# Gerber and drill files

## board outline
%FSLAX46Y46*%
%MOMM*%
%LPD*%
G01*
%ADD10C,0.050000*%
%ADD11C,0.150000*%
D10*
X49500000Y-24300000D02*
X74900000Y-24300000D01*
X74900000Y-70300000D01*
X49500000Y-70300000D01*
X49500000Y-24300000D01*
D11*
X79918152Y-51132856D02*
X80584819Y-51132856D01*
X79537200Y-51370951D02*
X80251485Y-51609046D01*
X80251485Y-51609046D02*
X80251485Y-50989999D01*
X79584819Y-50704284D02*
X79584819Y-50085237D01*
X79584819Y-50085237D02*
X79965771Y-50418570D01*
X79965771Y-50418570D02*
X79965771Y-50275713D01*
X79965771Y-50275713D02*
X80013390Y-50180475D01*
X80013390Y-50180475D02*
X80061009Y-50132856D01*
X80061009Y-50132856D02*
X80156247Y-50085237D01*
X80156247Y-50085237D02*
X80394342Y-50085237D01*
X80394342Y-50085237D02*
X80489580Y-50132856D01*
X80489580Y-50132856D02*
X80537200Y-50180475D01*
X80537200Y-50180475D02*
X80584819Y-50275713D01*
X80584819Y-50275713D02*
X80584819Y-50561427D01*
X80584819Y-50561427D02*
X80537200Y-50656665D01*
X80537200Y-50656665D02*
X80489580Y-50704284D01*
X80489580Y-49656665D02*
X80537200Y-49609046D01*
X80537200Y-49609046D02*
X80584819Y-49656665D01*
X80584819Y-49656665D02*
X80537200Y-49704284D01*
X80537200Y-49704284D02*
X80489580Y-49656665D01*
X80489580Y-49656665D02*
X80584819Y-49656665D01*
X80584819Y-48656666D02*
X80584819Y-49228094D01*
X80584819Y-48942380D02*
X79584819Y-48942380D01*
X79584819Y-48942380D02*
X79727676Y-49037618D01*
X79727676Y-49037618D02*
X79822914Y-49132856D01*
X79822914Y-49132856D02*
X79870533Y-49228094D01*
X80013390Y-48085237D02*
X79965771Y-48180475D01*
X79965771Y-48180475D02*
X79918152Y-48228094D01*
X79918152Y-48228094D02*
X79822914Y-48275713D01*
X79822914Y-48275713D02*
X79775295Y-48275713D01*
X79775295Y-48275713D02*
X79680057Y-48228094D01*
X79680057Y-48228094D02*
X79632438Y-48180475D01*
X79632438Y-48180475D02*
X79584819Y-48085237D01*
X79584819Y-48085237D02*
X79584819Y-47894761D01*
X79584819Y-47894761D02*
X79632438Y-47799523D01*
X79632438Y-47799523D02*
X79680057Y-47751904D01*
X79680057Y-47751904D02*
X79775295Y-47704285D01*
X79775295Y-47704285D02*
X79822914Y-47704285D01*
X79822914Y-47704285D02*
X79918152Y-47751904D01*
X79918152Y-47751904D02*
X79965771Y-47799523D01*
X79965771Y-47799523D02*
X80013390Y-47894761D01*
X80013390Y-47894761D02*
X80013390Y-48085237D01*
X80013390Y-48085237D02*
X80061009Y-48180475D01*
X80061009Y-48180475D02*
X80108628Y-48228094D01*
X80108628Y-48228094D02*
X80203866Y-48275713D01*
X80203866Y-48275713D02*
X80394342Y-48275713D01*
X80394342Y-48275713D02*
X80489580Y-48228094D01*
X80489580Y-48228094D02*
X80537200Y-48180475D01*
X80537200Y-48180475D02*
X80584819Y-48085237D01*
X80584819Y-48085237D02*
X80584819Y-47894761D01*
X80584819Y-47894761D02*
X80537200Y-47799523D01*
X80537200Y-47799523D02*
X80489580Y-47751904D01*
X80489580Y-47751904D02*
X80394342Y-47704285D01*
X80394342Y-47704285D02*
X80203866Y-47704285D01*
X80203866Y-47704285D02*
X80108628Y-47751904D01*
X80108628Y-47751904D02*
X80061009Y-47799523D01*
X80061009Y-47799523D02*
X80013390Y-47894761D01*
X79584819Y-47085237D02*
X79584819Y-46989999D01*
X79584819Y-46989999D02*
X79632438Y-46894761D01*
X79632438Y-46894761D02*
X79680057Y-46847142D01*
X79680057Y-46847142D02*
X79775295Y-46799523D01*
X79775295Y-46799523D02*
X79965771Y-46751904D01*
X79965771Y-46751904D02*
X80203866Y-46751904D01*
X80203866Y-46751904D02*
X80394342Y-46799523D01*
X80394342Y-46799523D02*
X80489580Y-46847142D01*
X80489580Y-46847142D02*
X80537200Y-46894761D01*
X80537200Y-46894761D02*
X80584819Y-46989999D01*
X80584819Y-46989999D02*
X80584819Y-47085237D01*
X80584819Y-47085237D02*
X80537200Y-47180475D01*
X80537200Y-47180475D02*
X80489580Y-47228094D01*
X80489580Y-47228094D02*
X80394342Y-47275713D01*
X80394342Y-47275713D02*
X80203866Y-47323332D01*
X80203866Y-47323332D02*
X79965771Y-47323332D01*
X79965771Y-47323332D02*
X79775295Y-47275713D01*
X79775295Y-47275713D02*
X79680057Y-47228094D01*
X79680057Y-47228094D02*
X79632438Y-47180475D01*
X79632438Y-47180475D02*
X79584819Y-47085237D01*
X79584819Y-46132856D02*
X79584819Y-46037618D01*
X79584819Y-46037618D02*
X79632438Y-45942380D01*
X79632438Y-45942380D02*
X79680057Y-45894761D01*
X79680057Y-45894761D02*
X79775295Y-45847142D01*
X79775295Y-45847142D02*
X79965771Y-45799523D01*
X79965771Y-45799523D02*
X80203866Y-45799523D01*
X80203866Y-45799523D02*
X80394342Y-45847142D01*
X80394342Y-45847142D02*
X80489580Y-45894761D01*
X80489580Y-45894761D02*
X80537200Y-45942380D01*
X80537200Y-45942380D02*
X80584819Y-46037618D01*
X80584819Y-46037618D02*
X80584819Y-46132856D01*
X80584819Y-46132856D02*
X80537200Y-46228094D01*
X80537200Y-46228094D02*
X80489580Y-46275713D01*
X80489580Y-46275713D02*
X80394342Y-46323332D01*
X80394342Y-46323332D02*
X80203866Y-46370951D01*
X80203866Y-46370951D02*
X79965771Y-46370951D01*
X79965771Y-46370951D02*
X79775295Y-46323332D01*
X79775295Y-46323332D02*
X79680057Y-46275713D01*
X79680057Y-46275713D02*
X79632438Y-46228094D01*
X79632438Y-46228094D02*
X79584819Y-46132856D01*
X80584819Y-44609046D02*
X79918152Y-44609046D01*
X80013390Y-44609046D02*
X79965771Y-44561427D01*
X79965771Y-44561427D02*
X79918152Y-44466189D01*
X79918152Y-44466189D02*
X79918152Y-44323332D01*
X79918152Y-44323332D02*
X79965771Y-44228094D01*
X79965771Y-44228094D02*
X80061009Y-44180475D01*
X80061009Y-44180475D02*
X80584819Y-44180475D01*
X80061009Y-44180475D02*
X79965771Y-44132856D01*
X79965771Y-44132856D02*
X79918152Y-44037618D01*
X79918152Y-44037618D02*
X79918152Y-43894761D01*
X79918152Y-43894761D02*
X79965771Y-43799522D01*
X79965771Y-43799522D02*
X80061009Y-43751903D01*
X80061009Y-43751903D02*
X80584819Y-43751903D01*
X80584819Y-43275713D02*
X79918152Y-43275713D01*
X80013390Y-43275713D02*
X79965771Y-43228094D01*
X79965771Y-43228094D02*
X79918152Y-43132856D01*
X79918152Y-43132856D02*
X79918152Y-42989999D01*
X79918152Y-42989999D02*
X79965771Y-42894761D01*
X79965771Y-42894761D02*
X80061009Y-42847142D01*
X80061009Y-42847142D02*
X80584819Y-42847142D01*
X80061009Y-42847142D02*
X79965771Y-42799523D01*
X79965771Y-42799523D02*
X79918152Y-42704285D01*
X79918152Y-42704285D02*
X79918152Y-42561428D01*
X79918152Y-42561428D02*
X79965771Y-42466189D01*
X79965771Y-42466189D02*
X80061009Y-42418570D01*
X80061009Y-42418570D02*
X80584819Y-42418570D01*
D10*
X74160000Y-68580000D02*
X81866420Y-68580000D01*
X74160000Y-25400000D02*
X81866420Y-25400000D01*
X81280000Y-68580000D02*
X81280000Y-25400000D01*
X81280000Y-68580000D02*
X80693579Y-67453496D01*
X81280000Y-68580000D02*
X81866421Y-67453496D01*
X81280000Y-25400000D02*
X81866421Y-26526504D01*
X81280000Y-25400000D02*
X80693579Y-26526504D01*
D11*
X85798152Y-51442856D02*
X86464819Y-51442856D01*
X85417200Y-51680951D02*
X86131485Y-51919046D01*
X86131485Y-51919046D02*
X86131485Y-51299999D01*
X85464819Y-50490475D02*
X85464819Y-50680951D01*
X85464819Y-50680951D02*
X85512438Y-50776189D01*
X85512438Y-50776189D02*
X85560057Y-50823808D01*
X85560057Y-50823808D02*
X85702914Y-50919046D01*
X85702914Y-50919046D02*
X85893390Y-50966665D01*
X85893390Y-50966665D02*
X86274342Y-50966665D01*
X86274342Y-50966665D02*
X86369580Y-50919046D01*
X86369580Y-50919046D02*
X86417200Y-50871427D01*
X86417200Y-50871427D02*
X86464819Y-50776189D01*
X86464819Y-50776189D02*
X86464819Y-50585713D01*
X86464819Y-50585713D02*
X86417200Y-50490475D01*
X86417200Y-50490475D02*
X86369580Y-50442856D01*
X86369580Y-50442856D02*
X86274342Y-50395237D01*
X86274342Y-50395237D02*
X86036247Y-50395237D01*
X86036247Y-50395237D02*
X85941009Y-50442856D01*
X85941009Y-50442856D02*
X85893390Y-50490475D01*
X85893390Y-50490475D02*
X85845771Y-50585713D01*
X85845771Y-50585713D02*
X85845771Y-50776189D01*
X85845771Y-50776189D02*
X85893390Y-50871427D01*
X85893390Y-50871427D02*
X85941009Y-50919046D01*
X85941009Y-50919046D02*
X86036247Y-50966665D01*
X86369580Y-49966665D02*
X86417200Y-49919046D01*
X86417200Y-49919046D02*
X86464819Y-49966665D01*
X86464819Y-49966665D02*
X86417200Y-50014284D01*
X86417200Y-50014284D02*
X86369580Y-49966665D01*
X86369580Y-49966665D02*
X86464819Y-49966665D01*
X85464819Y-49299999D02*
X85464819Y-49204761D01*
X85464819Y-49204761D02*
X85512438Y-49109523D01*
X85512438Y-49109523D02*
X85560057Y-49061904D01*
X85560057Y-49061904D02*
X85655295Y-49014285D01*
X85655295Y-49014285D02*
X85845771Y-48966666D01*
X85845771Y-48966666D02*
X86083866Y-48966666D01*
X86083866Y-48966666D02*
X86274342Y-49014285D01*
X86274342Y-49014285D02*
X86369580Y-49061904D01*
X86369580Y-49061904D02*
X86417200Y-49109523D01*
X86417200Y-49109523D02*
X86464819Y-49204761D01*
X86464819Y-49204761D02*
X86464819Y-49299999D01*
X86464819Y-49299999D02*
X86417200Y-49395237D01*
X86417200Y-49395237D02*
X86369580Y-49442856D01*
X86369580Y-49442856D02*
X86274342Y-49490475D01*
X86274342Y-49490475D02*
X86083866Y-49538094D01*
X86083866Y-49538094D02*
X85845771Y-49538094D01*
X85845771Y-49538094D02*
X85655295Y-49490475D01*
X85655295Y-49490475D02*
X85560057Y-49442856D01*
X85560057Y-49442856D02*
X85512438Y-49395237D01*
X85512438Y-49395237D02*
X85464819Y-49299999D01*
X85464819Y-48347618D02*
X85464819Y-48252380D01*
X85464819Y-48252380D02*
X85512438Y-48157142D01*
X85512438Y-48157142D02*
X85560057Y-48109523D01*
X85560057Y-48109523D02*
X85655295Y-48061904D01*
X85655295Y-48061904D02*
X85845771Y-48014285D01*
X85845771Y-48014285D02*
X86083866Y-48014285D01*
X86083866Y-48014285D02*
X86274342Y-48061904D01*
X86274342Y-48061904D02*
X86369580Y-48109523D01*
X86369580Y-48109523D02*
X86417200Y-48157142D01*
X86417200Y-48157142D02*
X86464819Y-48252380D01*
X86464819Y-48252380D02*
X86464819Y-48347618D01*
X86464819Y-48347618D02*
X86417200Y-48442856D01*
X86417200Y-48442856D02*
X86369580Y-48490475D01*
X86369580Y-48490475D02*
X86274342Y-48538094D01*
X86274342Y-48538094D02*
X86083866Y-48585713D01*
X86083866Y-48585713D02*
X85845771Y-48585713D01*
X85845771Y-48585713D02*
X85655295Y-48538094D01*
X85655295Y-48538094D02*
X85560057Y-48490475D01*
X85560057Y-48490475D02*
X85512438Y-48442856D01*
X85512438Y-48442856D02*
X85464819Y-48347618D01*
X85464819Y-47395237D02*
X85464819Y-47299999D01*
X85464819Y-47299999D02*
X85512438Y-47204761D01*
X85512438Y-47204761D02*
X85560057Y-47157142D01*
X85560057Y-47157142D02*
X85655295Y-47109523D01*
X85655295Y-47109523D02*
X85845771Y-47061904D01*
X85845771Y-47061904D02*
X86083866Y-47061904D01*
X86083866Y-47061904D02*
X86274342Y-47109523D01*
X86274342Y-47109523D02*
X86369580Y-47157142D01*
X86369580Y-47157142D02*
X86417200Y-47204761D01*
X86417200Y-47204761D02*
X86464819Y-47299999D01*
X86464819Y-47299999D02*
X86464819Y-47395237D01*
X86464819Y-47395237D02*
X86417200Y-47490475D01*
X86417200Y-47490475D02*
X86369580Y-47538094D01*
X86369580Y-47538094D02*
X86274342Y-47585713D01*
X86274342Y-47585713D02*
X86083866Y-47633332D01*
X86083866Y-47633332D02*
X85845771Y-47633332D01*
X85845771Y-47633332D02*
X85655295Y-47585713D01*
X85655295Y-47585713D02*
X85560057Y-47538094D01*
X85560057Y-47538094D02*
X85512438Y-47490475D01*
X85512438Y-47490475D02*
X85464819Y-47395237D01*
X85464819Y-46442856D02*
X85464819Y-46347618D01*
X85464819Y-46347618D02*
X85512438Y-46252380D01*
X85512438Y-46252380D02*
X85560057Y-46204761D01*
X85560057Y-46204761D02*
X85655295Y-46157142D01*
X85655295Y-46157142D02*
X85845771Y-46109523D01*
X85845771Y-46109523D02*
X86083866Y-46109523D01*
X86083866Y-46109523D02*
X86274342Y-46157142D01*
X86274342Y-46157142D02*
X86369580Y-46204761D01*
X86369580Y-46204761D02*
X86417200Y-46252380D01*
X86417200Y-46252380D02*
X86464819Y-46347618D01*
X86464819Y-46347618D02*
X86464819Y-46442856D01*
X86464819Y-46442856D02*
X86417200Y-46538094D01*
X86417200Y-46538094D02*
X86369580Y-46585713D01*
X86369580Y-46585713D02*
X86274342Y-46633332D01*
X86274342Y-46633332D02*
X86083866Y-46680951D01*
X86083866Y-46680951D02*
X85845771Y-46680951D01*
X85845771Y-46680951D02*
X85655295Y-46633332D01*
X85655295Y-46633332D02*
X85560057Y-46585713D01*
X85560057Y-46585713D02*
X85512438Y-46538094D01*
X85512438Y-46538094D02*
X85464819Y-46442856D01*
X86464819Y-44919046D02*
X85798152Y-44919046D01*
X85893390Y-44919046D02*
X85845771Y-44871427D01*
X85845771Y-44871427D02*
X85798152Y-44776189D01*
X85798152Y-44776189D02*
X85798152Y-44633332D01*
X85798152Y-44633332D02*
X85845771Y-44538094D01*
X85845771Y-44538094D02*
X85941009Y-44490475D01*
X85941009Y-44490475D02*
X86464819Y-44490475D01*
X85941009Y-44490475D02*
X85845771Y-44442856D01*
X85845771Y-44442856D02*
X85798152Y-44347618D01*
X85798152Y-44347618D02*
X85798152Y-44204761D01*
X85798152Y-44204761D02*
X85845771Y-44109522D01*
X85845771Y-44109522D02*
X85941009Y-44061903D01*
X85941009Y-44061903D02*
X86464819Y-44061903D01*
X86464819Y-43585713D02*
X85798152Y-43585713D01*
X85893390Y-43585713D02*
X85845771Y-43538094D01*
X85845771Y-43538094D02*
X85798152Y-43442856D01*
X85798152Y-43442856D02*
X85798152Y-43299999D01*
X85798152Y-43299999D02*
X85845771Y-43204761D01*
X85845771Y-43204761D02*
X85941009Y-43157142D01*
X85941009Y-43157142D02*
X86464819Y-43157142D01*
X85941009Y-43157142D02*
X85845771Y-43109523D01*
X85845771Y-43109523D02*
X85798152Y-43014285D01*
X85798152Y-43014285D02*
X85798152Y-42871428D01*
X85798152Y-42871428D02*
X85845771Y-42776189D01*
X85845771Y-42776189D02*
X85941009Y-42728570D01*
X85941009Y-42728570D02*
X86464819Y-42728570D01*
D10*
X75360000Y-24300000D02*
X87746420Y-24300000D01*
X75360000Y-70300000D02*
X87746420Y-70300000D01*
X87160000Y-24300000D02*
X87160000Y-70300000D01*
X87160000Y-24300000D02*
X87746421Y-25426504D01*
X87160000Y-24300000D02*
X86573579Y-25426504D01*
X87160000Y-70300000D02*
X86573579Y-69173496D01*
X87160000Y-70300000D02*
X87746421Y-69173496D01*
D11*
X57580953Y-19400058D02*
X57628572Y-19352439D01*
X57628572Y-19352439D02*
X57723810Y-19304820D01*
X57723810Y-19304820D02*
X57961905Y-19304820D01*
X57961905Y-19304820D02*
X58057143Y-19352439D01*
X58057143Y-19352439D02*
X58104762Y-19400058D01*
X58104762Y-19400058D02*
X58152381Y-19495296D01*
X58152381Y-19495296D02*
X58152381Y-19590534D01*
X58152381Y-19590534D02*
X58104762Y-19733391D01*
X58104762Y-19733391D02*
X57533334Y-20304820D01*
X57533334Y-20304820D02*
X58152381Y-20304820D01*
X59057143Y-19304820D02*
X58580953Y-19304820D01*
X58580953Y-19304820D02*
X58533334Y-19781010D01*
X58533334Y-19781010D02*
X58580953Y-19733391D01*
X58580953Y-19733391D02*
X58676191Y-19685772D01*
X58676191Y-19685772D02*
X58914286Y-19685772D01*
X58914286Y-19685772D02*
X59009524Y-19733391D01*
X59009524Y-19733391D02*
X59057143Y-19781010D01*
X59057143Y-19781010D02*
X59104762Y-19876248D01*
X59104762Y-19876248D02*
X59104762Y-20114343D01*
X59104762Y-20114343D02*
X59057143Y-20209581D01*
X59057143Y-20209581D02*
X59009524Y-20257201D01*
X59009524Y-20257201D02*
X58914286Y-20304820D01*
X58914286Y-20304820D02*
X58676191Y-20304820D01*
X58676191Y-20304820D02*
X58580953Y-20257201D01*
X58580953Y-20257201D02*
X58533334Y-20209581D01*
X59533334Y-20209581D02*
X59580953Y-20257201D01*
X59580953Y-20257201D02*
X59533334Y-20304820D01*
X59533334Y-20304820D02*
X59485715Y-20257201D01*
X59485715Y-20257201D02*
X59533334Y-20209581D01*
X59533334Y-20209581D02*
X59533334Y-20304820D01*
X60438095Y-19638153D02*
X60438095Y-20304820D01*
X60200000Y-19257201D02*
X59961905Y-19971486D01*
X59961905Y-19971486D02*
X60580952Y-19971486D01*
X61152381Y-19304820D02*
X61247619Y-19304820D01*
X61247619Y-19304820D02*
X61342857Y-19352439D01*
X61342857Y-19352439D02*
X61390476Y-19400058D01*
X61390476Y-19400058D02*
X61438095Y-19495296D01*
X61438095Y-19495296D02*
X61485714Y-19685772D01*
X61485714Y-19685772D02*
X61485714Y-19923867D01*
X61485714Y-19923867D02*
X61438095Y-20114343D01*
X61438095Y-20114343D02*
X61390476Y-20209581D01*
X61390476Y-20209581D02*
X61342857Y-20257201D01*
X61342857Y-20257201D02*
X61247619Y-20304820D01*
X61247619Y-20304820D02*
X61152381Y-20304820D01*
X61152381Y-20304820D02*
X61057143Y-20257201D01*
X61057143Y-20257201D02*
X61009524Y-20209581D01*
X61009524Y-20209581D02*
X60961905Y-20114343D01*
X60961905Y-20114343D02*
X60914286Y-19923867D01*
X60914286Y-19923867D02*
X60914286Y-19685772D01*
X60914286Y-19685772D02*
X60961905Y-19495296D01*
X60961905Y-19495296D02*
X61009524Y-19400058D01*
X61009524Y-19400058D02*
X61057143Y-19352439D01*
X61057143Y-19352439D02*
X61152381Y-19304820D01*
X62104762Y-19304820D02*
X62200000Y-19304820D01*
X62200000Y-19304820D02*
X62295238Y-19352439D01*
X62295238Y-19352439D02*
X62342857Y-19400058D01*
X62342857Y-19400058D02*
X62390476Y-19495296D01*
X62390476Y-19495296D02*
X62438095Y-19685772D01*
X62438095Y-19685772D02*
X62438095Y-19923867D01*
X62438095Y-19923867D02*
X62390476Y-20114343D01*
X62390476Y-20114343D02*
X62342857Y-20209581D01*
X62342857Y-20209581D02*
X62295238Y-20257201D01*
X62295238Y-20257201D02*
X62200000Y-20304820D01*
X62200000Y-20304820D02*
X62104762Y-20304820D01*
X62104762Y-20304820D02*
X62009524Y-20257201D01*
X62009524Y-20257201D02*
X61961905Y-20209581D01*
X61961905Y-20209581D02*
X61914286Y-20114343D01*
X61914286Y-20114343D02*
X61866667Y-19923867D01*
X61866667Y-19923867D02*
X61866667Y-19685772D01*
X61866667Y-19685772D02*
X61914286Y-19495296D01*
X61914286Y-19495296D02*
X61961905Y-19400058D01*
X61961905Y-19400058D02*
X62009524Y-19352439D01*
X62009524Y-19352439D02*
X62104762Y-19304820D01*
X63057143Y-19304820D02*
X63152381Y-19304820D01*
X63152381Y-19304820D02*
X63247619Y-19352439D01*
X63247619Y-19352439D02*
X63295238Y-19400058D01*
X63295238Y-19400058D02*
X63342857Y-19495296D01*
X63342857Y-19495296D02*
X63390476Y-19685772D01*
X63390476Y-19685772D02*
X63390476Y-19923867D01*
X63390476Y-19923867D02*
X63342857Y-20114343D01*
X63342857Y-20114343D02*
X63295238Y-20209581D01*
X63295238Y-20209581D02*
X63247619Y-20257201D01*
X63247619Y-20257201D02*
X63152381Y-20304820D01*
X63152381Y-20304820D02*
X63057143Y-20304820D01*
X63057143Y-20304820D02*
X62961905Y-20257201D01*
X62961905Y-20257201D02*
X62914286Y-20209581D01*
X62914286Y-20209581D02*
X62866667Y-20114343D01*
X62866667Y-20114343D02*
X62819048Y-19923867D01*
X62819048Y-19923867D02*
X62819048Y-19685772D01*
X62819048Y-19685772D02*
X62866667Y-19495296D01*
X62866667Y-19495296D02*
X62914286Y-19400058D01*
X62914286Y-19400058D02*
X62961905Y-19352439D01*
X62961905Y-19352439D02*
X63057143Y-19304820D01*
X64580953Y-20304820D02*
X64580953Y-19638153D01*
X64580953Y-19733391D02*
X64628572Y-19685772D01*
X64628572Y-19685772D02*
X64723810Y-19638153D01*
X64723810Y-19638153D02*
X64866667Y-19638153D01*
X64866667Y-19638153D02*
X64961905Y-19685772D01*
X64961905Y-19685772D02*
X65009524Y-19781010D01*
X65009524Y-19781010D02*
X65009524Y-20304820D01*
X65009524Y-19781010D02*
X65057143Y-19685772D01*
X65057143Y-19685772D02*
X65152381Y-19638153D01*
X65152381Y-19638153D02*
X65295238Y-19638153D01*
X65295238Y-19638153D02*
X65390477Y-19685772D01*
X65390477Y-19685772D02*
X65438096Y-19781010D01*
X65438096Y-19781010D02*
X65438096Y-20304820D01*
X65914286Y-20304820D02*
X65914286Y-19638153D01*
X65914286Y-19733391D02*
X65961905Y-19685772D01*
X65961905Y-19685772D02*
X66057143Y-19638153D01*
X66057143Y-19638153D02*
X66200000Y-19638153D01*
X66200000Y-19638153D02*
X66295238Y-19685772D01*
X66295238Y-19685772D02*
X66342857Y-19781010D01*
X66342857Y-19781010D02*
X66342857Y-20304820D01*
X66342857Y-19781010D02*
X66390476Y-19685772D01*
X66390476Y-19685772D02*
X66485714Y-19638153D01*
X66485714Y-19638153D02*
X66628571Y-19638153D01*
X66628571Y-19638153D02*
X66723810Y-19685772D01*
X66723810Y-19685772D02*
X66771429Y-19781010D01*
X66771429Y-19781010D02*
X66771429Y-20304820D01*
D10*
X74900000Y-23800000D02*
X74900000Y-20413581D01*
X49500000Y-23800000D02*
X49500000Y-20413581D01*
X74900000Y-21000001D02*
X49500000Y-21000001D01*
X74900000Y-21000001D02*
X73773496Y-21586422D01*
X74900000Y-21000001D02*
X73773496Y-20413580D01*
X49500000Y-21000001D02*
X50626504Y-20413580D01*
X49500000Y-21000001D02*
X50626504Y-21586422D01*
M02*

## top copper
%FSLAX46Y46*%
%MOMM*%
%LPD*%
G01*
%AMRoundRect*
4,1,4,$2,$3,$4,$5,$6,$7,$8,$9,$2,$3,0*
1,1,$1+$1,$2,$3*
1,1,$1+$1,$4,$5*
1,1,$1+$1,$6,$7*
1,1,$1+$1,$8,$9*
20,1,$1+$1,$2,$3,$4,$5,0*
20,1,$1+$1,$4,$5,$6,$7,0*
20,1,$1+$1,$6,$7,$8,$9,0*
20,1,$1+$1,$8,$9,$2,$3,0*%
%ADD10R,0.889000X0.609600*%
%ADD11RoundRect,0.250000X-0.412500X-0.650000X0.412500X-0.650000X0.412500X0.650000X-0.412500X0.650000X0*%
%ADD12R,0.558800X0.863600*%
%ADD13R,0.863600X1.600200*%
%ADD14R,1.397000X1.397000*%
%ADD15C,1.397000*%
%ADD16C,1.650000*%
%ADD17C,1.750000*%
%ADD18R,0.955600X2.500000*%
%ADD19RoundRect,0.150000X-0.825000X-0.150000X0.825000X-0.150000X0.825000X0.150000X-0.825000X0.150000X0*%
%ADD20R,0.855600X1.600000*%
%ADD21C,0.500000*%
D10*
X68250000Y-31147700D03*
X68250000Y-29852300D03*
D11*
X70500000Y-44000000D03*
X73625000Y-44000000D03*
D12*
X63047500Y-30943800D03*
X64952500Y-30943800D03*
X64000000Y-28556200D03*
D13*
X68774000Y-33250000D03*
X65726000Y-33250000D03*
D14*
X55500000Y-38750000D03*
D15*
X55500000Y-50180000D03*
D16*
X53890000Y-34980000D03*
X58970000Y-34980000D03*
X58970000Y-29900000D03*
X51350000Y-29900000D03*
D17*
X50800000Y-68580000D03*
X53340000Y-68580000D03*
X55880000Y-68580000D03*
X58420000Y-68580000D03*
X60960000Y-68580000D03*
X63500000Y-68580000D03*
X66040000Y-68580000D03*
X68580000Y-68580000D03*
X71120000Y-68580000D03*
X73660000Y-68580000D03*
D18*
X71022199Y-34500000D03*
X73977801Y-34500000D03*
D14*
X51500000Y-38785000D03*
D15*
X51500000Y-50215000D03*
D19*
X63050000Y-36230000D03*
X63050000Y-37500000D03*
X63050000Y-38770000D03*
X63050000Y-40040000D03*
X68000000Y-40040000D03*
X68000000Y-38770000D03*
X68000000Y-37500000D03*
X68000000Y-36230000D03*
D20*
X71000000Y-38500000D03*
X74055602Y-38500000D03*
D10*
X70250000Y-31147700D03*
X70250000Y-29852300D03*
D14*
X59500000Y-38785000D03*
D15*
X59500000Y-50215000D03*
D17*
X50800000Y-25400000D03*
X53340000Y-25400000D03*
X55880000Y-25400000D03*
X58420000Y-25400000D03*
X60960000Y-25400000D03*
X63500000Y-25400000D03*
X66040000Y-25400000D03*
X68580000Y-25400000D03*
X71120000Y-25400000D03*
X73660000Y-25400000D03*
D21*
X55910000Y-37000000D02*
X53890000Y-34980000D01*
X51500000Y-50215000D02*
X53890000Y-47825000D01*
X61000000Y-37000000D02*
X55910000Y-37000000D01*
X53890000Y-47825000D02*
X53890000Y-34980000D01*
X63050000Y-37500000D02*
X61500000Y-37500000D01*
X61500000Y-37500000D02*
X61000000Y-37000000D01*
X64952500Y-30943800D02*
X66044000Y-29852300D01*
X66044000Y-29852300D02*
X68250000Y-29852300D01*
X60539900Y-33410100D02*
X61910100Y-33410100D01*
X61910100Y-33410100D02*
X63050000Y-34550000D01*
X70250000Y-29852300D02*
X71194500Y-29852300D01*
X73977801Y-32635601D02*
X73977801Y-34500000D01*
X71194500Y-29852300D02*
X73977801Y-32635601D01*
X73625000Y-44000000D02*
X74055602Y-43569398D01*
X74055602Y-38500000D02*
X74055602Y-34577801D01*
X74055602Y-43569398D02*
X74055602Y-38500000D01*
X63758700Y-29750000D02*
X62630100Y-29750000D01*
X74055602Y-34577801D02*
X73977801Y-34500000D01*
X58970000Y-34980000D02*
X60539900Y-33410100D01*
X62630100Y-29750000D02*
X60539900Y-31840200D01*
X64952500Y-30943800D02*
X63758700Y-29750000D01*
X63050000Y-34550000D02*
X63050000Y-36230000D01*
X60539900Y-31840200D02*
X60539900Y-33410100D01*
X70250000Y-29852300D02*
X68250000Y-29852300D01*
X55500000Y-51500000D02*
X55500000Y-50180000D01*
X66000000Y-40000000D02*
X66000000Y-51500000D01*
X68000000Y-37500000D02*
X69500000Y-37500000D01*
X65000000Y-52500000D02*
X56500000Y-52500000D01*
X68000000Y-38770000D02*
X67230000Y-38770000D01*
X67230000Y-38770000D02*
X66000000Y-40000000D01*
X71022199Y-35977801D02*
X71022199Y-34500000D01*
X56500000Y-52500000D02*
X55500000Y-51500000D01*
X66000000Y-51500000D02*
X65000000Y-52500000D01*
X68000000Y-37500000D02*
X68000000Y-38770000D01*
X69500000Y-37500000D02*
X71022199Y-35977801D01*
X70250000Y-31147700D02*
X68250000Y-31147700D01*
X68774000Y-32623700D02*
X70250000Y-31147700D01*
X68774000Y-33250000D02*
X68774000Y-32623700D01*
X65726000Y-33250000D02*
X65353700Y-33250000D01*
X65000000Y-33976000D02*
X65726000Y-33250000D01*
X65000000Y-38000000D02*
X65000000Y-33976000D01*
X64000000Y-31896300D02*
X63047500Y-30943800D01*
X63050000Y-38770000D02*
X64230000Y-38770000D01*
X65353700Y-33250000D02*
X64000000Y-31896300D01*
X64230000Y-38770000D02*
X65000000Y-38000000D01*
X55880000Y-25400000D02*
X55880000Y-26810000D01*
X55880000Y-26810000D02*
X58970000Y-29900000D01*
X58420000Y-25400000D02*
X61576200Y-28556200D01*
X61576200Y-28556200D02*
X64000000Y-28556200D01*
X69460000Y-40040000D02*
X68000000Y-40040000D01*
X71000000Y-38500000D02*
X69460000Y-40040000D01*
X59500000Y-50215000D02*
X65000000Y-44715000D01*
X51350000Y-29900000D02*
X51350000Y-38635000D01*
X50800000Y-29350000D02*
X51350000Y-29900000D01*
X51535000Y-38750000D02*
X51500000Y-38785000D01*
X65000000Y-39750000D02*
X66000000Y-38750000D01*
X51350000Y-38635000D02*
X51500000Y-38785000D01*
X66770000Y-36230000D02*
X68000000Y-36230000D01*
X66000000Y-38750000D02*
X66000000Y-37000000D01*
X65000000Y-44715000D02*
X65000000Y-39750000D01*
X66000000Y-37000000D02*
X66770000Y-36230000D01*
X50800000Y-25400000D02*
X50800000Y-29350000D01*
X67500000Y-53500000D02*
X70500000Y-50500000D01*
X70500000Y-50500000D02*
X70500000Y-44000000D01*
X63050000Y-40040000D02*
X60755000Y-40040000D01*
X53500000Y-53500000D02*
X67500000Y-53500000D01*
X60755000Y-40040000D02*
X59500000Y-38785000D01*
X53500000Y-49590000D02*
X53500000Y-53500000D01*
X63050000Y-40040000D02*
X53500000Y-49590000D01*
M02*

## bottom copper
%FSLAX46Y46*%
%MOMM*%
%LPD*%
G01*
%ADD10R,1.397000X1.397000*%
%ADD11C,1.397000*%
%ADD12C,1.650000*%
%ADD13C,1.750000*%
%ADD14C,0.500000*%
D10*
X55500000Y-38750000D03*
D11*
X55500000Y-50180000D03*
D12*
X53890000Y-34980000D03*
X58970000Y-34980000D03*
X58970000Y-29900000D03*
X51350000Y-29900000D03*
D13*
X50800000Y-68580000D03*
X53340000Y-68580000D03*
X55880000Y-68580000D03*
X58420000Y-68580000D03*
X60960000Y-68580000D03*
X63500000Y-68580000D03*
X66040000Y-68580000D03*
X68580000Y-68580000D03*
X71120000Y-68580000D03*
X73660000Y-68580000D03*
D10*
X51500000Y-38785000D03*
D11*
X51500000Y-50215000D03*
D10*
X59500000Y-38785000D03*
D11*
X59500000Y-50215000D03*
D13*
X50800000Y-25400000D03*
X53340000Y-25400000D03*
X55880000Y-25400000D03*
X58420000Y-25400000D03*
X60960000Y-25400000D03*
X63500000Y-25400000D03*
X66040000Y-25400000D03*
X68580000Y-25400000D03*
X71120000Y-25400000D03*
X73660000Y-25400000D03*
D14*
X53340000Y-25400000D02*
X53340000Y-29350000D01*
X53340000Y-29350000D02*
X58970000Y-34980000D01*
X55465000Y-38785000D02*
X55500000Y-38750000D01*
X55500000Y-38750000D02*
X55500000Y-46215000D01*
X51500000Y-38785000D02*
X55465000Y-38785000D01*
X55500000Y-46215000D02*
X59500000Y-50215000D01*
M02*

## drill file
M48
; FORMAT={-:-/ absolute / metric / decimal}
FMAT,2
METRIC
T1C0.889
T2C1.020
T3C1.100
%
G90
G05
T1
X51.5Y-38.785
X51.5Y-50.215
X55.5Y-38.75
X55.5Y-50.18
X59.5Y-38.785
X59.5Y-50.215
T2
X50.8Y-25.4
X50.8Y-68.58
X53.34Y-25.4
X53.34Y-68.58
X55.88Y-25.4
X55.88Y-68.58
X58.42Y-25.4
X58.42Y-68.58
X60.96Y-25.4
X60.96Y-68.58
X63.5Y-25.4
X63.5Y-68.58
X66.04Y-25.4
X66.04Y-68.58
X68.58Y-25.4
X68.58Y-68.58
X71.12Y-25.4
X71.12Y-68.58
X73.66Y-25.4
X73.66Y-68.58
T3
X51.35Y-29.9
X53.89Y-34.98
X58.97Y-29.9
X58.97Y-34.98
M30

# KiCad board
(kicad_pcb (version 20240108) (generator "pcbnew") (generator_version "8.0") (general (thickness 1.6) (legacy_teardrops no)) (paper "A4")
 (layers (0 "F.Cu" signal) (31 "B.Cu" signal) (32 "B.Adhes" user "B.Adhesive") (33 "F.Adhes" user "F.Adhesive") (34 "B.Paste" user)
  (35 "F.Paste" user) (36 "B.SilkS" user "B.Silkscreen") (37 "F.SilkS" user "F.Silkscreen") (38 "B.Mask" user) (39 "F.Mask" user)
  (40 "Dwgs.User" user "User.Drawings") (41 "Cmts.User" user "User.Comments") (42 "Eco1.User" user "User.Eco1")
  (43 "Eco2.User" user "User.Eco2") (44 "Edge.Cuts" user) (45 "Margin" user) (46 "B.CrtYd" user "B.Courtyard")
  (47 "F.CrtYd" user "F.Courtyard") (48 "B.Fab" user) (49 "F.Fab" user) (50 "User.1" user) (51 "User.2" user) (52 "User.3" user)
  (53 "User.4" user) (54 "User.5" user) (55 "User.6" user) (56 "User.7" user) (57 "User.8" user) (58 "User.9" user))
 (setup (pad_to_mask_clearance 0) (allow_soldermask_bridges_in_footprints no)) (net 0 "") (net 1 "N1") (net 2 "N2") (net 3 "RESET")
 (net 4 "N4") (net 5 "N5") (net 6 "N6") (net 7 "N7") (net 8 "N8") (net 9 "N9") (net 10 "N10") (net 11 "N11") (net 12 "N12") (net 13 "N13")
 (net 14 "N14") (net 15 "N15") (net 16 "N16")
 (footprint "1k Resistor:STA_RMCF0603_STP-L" (layer "F.Cu") (at 68.25 30.5 90)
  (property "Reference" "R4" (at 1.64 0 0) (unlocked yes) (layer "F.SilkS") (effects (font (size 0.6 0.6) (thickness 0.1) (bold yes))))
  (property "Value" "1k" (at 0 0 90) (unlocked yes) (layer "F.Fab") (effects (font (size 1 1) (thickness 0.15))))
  (pad "1" smd rect (at -0.6477 0 90) (size 0.6096 0.889) (layers "F.Cu" "F.Paste" "F.Mask") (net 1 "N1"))
  (pad "2" smd rect (at 0.6477 0 90) (size 0.6096 0.889) (layers "F.Cu" "F.Paste" "F.Mask") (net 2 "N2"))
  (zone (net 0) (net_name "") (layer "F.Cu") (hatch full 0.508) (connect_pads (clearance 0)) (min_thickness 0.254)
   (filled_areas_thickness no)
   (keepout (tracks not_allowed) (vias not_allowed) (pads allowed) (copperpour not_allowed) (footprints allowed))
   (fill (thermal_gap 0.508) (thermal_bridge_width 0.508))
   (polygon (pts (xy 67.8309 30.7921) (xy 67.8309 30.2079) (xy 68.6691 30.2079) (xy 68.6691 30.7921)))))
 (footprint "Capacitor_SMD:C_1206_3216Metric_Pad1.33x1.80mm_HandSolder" (layer "F.Cu") (at 72.0625 44)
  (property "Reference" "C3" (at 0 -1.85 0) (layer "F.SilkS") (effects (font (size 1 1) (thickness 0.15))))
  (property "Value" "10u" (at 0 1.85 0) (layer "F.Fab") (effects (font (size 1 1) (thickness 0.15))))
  (pad "1" smd roundrect (at -1.5625 0) (size 1.325 1.8) (layers "F.Cu" "F.Paste" "F.Mask") (roundrect_rratio 0.188679) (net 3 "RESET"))
  (pad "2" smd roundrect (at 1.5625 0) (size 1.325 1.8) (layers "F.Cu" "F.Paste" "F.Mask") (roundrect_rratio 0.188679) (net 2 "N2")))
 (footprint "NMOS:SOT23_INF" (layer "F.Cu") (at 64 29.75)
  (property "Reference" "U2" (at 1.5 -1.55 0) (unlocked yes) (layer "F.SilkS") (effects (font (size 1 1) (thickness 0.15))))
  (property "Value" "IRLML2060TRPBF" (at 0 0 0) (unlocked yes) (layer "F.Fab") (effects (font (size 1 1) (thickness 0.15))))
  (pad "1" smd rect (at -0.9525 1.1938) (size 0.5588 0.8636) (layers "F.Cu" "F.Paste" "F.Mask") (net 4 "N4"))
  (pad "2" smd rect (at 0.9525 1.1938) (size 0.5588 0.8636) (layers "F.Cu" "F.Paste" "F.Mask") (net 2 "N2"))
  (pad "3" smd rect (at 0 -1.1938) (size 0.5588 0.8636) (layers "F.Cu" "F.Paste" "F.Mask") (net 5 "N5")))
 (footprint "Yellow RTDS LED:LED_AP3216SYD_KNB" (layer "F.Cu") (at 67.25 33.25 180)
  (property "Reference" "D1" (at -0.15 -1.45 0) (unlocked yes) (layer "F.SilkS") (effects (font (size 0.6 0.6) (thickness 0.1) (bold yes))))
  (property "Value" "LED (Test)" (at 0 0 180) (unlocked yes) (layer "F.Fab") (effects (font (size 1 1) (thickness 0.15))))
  (pad "1" smd rect (at -1.524 0 180) (size 0.8636 1.6002) (layers "F.Cu" "F.Paste" "F.Mask") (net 1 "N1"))
  (pad "2" smd rect (at 1.524 0 180) (size 0.8636 1.6002) (layers "F.Cu" "F.Paste" "F.Mask") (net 4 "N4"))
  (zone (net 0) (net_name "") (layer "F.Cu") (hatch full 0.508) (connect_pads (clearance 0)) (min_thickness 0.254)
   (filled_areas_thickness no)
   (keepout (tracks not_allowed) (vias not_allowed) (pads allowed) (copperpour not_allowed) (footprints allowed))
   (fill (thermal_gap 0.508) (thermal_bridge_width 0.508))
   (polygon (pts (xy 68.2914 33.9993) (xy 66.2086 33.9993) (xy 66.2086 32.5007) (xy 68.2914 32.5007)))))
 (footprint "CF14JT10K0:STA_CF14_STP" (layer "F.Cu") (at 55.5 38.75 -90)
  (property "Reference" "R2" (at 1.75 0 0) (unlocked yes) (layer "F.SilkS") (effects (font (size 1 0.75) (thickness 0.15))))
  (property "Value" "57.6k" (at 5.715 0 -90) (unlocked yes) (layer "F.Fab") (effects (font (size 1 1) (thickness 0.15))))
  (pad "1" thru_hole rect (at 0 0 270) (size 1.397 1.397) (drill 0.889) (layers "*.Cu" "*.Mask") (remove_unused_layers no) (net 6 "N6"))
  (pad "2" thru_hole circle (at 11.43 0 270) (size 1.397 1.397) (drill 0.889) (layers "*.Cu" "*.Mask") (remove_unused_layers no)
   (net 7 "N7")))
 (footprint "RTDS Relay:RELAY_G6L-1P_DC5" (layer "F.Cu") (at 55.16 32.44)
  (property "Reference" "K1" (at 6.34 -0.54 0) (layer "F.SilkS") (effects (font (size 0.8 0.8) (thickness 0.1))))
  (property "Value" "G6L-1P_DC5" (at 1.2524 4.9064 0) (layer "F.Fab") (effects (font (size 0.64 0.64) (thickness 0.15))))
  (pad "2" thru_hole circle (at -1.27 2.54) (size 1.65 1.65) (drill 1.1) (layers "*.Cu" "*.Mask") (remove_unused_layers no) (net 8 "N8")
   (solder_mask_margin 0.102))
  (pad "4" thru_hole circle (at 3.81 2.54) (size 1.65 1.65) (drill 1.1) (layers "*.Cu" "*.Mask") (remove_unused_layers no) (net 2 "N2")
   (solder_mask_margin 0.102))
  (pad "5" thru_hole circle (at 3.81 -2.54) (size 1.65 1.65) (drill 1.1) (layers "*.Cu" "*.Mask") (remove_unused_layers no) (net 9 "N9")
   (solder_mask_margin 0.102))
  (pad "8" thru_hole circle (at -3.81 -2.54) (size 1.65 1.65) (drill 1.1) (layers "*.Cu" "*.Mask") (remove_unused_layers no) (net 6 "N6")
   (solder_mask_margin 0.102)))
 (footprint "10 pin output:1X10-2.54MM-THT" (layer "F.Cu") (at 50.8 68.58)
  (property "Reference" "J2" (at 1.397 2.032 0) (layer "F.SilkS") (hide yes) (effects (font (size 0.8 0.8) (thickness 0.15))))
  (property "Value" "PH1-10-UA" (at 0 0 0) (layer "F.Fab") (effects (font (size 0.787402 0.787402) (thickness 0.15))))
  (pad "1" thru_hole circle (at 0 0) (size 1.75 1.75) (drill 1.02) (layers "*.Cu" "*.Mask") (remove_unused_layers no)
   (solder_mask_margin 0.102))
  (pad "2" thru_hole circle (at 2.54 0) (size 1.75 1.75) (drill 1.02) (layers "*.Cu" "*.Mask") (remove_unused_layers no)
   (solder_mask_margin 0.102))
  (pad "3" thru_hole circle (at 5.08 0) (size 1.75 1.75) (drill 1.02) (layers "*.Cu" "*.Mask") (remove_unused_layers no)
   (solder_mask_margin 0.102))
  (pad "4" thru_hole circle (at 7.62 0) (size 1.75 1.75) (drill 1.02) (layers "*.Cu" "*.Mask") (remove_unused_layers no)
   (solder_mask_margin 0.102))
  (pad "5" thru_hole circle (at 10.16 0) (size 1.75 1.75) (drill 1.02) (layers "*.Cu" "*.Mask") (remove_unused_layers no)
   (solder_mask_margin 0.102))
  (pad "6" thru_hole circle (at 12.7 0) (size 1.75 1.75) (drill 1.02) (layers "*.Cu" "*.Mask") (remove_unused_layers no)
   (solder_mask_margin 0.102))
  (pad "7" thru_hole circle (at 15.24 0) (size 1.75 1.75) (drill 1.02) (layers "*.Cu" "*.Mask") (remove_unused_layers no)
   (solder_mask_margin 0.102))
  (pad "8" thru_hole circle (at 17.78 0) (size 1.75 1.75) (drill 1.02) (layers "*.Cu" "*.Mask") (remove_unused_layers no)
   (solder_mask_margin 0.102))
  (pad "9" thru_hole circle (at 20.32 0) (size 1.75 1.75) (drill 1.02) (layers "*.Cu" "*.Mask") (remove_unused_layers no)
   (solder_mask_margin 0.102))
  (pad "10" thru_hole circle (at 22.86 0) (size 1.75 1.75) (drill 1.02) (layers "*.Cu" "*.Mask") (remove_unused_layers no)
   (solder_mask_margin 0.102)))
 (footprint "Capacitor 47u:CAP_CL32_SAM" (layer "F.Cu") (at 72.5 34.5)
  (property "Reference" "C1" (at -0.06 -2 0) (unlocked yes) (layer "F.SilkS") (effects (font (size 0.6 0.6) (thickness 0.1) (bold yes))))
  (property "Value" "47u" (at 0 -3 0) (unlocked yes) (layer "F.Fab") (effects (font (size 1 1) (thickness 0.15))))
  (pad "1" smd rect (at -1.477801 0) (size 0.9556 2.5) (layers "F.Cu" "F.Paste" "F.Mask") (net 7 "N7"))
  (pad "2" smd rect (at 1.477801 0) (size 0.9556 2.5) (layers "F.Cu" "F.Paste" "F.Mask") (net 2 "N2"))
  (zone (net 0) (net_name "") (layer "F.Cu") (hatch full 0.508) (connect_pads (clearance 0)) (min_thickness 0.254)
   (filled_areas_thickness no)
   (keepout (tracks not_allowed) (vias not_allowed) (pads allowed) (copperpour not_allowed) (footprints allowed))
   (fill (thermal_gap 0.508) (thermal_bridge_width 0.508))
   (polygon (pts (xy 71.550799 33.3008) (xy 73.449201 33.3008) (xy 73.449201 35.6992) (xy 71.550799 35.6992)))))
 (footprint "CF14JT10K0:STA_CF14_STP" (layer "F.Cu") (at 51.5 38.785 -90)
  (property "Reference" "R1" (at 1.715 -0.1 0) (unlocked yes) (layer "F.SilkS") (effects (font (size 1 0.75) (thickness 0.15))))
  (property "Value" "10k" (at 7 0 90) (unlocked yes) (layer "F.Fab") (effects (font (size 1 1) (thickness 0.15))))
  (pad "1" thru_hole rect (at 0 0 270) (size 1.397 1.397) (drill 0.889) (layers "*.Cu" "*.Mask") (remove_unused_layers no) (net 6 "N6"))
  (pad "2" thru_hole circle (at 11.43 0 270) (size 1.397 1.397) (drill 0.889) (layers "*.Cu" "*.Mask") (remove_unused_layers no)
   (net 8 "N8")))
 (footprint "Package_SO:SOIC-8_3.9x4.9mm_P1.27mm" (layer "F.Cu") (at 65.525 38.135)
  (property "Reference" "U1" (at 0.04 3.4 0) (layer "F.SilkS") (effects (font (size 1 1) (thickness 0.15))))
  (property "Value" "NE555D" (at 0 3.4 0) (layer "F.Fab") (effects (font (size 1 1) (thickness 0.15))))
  (pad "1" smd roundrect (at -2.475 -1.905) (size 1.95 0.6) (layers "F.Cu" "F.Paste" "F.Mask") (roundrect_rratio 0.25) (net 2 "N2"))
  (pad "2" smd roundrect (at -2.475 -0.635) (size 1.95 0.6) (layers "F.Cu" "F.Paste" "F.Mask") (roundrect_rratio 0.25) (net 8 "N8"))
  (pad "3" smd roundrect (at -2.475 0.635) (size 1.95 0.6) (layers "F.Cu" "F.Paste" "F.Mask") (roundrect_rratio 0.25) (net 4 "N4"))
  (pad "4" smd roundrect (at -2.475 1.905) (size 1.95 0.6) (layers "F.Cu" "F.Paste" "F.Mask") (roundrect_rratio 0.25) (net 3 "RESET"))
  (pad "5" smd roundrect (at 2.475 1.905) (size 1.95 0.6) (layers "F.Cu" "F.Paste" "F.Mask") (roundrect_rratio 0.25) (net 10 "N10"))
  (pad "6" smd roundrect (at 2.475 0.635) (size 1.95 0.6) (layers "F.Cu" "F.Paste" "F.Mask") (roundrect_rratio 0.25) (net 7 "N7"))
  (pad "7" smd roundrect (at 2.475 -0.635) (size 1.95 0.6) (layers "F.Cu" "F.Paste" "F.Mask") (roundrect_rratio 0.25) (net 7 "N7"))
  (pad "8" smd roundrect (at 2.475 -1.905) (size 1.95 0.6) (layers "F.Cu" "F.Paste" "F.Mask") (roundrect_rratio 0.25) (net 6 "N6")))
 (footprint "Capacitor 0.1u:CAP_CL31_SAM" (layer "F.Cu") (at 72.527801 38.5)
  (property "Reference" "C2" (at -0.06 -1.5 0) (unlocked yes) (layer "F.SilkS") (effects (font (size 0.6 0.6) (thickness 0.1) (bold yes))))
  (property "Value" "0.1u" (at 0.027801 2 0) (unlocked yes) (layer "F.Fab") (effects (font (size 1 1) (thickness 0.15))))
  (pad "1" smd rect (at -1.527801 0) (size 0.8556 1.6) (layers "F.Cu" "F.Paste" "F.Mask") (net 10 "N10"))
  (pad "2" smd rect (at 1.527801 0) (size 0.8556 1.6) (layers "F.Cu" "F.Paste" "F.Mask") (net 2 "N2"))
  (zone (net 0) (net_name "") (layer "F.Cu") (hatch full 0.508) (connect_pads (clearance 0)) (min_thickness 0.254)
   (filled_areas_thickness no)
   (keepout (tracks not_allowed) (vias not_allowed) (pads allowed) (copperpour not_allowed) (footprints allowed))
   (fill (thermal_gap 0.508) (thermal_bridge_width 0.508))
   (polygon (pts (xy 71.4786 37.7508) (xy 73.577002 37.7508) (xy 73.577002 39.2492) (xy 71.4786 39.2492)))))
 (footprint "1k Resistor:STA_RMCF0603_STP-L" (layer "F.Cu") (at 70.25 30.5 90)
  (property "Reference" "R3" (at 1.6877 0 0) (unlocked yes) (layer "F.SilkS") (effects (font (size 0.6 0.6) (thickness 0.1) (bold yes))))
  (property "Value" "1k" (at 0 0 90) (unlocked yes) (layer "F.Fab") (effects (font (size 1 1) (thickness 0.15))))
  (pad "1" smd rect (at -0.6477 0 90) (size 0.6096 0.889) (layers "F.Cu" "F.Paste" "F.Mask") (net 1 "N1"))
  (pad "2" smd rect (at 0.6477 0 90) (size 0.6096 0.889) (layers "F.Cu" "F.Paste" "F.Mask") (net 2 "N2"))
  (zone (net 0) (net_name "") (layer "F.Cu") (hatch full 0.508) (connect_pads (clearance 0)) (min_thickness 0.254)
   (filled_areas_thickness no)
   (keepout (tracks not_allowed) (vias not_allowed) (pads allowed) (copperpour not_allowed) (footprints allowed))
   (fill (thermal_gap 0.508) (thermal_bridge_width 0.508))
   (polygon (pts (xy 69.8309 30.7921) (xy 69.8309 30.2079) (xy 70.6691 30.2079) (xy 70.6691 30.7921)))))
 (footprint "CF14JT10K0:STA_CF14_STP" (layer "F.Cu") (at 59.5 38.785 -90)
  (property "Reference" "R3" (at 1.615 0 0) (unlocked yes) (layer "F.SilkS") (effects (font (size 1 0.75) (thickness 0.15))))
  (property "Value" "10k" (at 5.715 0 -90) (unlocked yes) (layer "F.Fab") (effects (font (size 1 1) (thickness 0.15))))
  (pad "1" thru_hole rect (at 0 0 270) (size 1.397 1.397) (drill 0.889) (layers "*.Cu" "*.Mask") (remove_unused_layers no) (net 3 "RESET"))
  (pad "2" thru_hole circle (at 11.43 0 270) (size 1.397 1.397) (drill 0.889) (layers "*.Cu" "*.Mask") (remove_unused_layers no)
   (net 6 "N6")))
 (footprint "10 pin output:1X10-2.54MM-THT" (layer "F.Cu") (at 50.8 25.4)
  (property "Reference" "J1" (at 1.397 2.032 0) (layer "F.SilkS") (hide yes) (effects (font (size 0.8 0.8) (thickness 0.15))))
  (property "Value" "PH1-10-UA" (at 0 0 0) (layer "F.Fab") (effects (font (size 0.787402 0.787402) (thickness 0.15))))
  (pad "1" thru_hole circle (at 0 0) (size 1.75 1.75) (drill 1.02) (layers "*.Cu" "*.Mask") (remove_unused_layers no) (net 6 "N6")
   (solder_mask_margin 0.102))
  (pad "2" thru_hole circle (at 2.54 0) (size 1.75 1.75) (drill 1.02) (layers "*.Cu" "*.Mask") (remove_unused_layers no) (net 2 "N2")
   (solder_mask_margin 0.102))
  (pad "3" thru_hole circle (at 5.08 0) (size 1.75 1.75) (drill 1.02) (layers "*.Cu" "*.Mask") (remove_unused_layers no) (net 9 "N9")
   (solder_mask_margin 0.102))
  (pad "4" thru_hole circle (at 7.62 0) (size 1.75 1.75) (drill 1.02) (layers "*.Cu" "*.Mask") (remove_unused_layers no) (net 5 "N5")
   (solder_mask_margin 0.102))
  (pad "5" thru_hole circle (at 10.16 0) (size 1.75 1.75) (drill 1.02) (layers "*.Cu" "*.Mask") (remove_unused_layers no) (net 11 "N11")
   (solder_mask_margin 0.102))
  (pad "6" thru_hole circle (at 12.7 0) (size 1.75 1.75) (drill 1.02) (layers "*.Cu" "*.Mask") (remove_unused_layers no) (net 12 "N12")
   (solder_mask_margin 0.102))
  (pad "7" thru_hole circle (at 15.24 0) (size 1.75 1.75) (drill 1.02) (layers "*.Cu" "*.Mask") (remove_unused_layers no) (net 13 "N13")
   (solder_mask_margin 0.102))
  (pad "8" thru_hole circle (at 17.78 0) (size 1.75 1.75) (drill 1.02) (layers "*.Cu" "*.Mask") (remove_unused_layers no) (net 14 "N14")
   (solder_mask_margin 0.102))
  (pad "9" thru_hole circle (at 20.32 0) (size 1.75 1.75) (drill 1.02) (layers "*.Cu" "*.Mask") (remove_unused_layers no) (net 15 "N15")
   (solder_mask_margin 0.102))
  (pad "10" thru_hole circle (at 22.86 0) (size 1.75 1.75) (drill 1.02) (layers "*.Cu" "*.Mask") (remove_unused_layers no) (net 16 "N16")
   (solder_mask_margin 0.102)))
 (gr_rect (start 49.5 24.3) (end 74.9 70.3) (stroke (width 0.05) (type default)) (fill none) (layer "Edge.Cuts"))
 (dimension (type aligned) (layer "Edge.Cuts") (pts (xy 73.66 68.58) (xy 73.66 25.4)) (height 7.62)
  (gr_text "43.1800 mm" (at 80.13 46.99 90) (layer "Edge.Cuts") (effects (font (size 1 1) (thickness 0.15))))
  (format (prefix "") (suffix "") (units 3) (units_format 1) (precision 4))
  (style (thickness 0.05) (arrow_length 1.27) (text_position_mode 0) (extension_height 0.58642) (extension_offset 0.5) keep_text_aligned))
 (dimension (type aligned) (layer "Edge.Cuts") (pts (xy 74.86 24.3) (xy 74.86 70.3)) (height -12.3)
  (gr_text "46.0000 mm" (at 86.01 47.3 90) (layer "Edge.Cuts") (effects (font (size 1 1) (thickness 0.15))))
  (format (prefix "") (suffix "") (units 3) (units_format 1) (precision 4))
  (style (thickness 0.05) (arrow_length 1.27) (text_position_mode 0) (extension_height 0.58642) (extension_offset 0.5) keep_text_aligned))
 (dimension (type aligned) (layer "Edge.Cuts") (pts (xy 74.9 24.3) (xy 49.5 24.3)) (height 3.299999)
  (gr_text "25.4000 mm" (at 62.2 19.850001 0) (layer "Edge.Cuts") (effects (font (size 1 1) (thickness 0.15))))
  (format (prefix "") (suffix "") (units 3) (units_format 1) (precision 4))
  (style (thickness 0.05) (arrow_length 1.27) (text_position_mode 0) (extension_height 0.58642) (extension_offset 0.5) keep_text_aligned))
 (segment (start 55.91 37) (end 53.89 34.98) (width 0.5) (layer "F.Cu") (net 8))
 (segment (start 51.5 50.215) (end 53.89 47.825) (width 0.5) (layer "F.Cu") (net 8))
 (segment (start 61 37) (end 55.91 37) (width 0.5) (layer "F.Cu") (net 8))
 (segment (start 53.89 47.825) (end 53.89 34.98) (width 0.5) (layer "F.Cu") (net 8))
 (segment (start 63.05 37.5) (end 61.5 37.5) (width 0.5) (layer "F.Cu") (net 8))
 (segment (start 61.5 37.5) (end 61 37) (width 0.5) (layer "F.Cu") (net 8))
 (segment (start 64.9525 30.9438) (end 66.044 29.8523) (width 0.5) (layer "F.Cu") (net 2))
 (segment (start 66.044 29.8523) (end 68.25 29.8523) (width 0.5) (layer "F.Cu") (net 2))
 (segment (start 60.5399 33.4101) (end 61.9101 33.4101) (width 0.5) (layer "F.Cu") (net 2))
 (segment (start 61.9101 33.4101) (end 63.05 34.55) (width 0.5) (layer "F.Cu") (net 2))
 (segment (start 70.25 29.8523) (end 71.1945 29.8523) (width 0.5) (layer "F.Cu") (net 2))
 (segment (start 73.977801 32.635601) (end 73.977801 34.5) (width 0.5) (layer "F.Cu") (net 2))
 (segment (start 71.1945 29.8523) (end 73.977801 32.635601) (width 0.5) (layer "F.Cu") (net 2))
 (segment (start 73.625 44) (end 74.055602 43.569398) (width 0.5) (layer "F.Cu") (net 2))
 (segment (start 74.055602 38.5) (end 74.055602 34.577801) (width 0.5) (layer "F.Cu") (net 2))
 (segment (start 74.055602 43.569398) (end 74.055602 38.5) (width 0.5) (layer "F.Cu") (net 2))
 (segment (start 63.7587 29.75) (end 62.6301 29.75) (width 0.5) (layer "F.Cu") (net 2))
 (segment (start 74.055602 34.577801) (end 73.977801 34.5) (width 0.5) (layer "F.Cu") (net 2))
 (segment (start 58.97 34.98) (end 60.5399 33.4101) (width 0.5) (layer "F.Cu") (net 2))
 (segment (start 62.6301 29.75) (end 60.5399 31.8402) (width 0.5) (layer "F.Cu") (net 2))
 (segment (start 64.9525 30.9438) (end 63.7587 29.75) (width 0.5) (layer "F.Cu") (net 2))
 (segment (start 63.05 34.55) (end 63.05 36.23) (width 0.5) (layer "F.Cu") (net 2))
 (segment (start 60.5399 31.8402) (end 60.5399 33.4101) (width 0.5) (layer "F.Cu") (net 2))
 (segment (start 70.25 29.8523) (end 68.25 29.8523) (width 0.5) (layer "F.Cu") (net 2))
 (segment (start 53.34 25.4) (end 53.34 29.35) (width 0.5) (layer "B.Cu") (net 2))
 (segment (start 53.34 29.35) (end 58.97 34.98) (width 0.5) (layer "B.Cu") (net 2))
 (segment (start 55.5 51.5) (end 55.5 50.18) (width 0.5) (layer "F.Cu") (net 7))
 (segment (start 66 40) (end 66 51.5) (width 0.5) (layer "F.Cu") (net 7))
 (segment (start 68 37.5) (end 69.5 37.5) (width 0.5) (layer "F.Cu") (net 7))
 (segment (start 65 52.5) (end 56.5 52.5) (width 0.5) (layer "F.Cu") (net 7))
 (segment (start 68 38.77) (end 67.23 38.77) (width 0.5) (layer "F.Cu") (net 7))
 (segment (start 67.23 38.77) (end 66 40) (width 0.5) (layer "F.Cu") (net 7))
 (segment (start 71.022199 35.977801) (end 71.022199 34.5) (width 0.5) (layer "F.Cu") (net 7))
 (segment (start 56.5 52.5) (end 55.5 51.5) (width 0.5) (layer "F.Cu") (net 7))
 (segment (start 66 51.5) (end 65 52.5) (width 0.5) (layer "F.Cu") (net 7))
 (segment (start 68 37.5) (end 68 38.77) (width 0.5) (layer "F.Cu") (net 7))
 (segment (start 69.5 37.5) (end 71.022199 35.977801) (width 0.5) (layer "F.Cu") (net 7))
 (segment (start 70.25 31.1477) (end 68.25 31.1477) (width 0.5) (layer "F.Cu") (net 1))
 (segment (start 68.774 32.6237) (end 70.25 31.1477) (width 0.5) (layer "F.Cu") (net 1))
 (segment (start 68.774 33.25) (end 68.774 32.6237) (width 0.5) (layer "F.Cu") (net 1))
 (segment (start 65.726 33.25) (end 65.3537 33.25) (width 0.5) (layer "F.Cu") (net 4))
 (segment (start 65 33.976) (end 65.726 33.25) (width 0.5) (layer "F.Cu") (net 4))
 (segment (start 65 38) (end 65 33.976) (width 0.5) (layer "F.Cu") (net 4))
 (segment (start 64 31.8963) (end 63.0475 30.9438) (width 0.5) (layer "F.Cu") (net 4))
 (segment (start 63.05 38.77) (end 64.23 38.77) (width 0.5) (layer "F.Cu") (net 4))
 (segment (start 65.3537 33.25) (end 64 31.8963) (width 0.5) (layer "F.Cu") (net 4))
 (segment (start 64.23 38.77) (end 65 38) (width 0.5) (layer "F.Cu") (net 4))
 (segment (start 55.88 25.4) (end 55.88 26.81) (width 0.5) (layer "F.Cu") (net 9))
 (segment (start 55.88 26.81) (end 58.97 29.9) (width 0.5) (layer "F.Cu") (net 9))
 (segment (start 58.42 25.4) (end 61.5762 28.5562) (width 0.5) (layer "F.Cu") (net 5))
 (segment (start 61.5762 28.5562) (end 64 28.5562) (width 0.5) (layer "F.Cu") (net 5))
 (segment (start 69.46 40.04) (end 68 40.04) (width 0.5) (layer "F.Cu") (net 10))
 (segment (start 71 38.5) (end 69.46 40.04) (width 0.5) (layer "F.Cu") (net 10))
 (segment (start 59.5 50.215) (end 65 44.715) (width 0.5) (layer "F.Cu") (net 6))
 (segment (start 51.35 29.9) (end 51.35 38.635) (width 0.5) (layer "F.Cu") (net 6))
 (segment (start 50.8 29.35) (end 51.35 29.9) (width 0.5) (layer "F.Cu") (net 6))
 (segment (start 51.535 38.75) (end 51.5 38.785) (width 0.5) (layer "F.Cu") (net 6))
 (segment (start 65 39.75) (end 66 38.75) (width 0.5) (layer "F.Cu") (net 6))
 (segment (start 51.35 38.635) (end 51.5 38.785) (width 0.5) (layer "F.Cu") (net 6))
 (segment (start 66.77 36.23) (end 68 36.23) (width 0.5) (layer "F.Cu") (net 6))
 (segment (start 66 38.75) (end 66 37) (width 0.5) (layer "F.Cu") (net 6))
 (segment (start 65 44.715) (end 65 39.75) (width 0.5) (layer "F.Cu") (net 6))
 (segment (start 66 37) (end 66.77 36.23) (width 0.5) (layer "F.Cu") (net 6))
 (segment (start 50.8 25.4) (end 50.8 29.35) (width 0.5) (layer "F.Cu") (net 6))
 (segment (start 55.465 38.785) (end 55.5 38.75) (width 0.5) (layer "B.Cu") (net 6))
 (segment (start 55.5 38.75) (end 55.5 46.215) (width 0.5) (layer "B.Cu") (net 6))
 (segment (start 51.5 38.785) (end 55.465 38.785) (width 0.5) (layer "B.Cu") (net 6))
 (segment (start 55.5 46.215) (end 59.5 50.215) (width 0.5) (layer "B.Cu") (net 6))
 (segment (start 67.5 53.5) (end 70.5 50.5) (width 0.5) (layer "F.Cu") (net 3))
 (segment (start 70.5 50.5) (end 70.5 44) (width 0.5) (layer "F.Cu") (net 3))
 (segment (start 63.05 40.04) (end 60.755 40.04) (width 0.5) (layer "F.Cu") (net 3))
 (segment (start 53.5 53.5) (end 67.5 53.5) (width 0.5) (layer "F.Cu") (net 3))
 (segment (start 60.755 40.04) (end 59.5 38.785) (width 0.5) (layer "F.Cu") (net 3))
 (segment (start 53.5 49.59) (end 53.5 53.5) (width 0.5) (layer "F.Cu") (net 3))
 (segment (start 63.05 40.04) (end 53.5 49.59) (width 0.5) (layer "F.Cu") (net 3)))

